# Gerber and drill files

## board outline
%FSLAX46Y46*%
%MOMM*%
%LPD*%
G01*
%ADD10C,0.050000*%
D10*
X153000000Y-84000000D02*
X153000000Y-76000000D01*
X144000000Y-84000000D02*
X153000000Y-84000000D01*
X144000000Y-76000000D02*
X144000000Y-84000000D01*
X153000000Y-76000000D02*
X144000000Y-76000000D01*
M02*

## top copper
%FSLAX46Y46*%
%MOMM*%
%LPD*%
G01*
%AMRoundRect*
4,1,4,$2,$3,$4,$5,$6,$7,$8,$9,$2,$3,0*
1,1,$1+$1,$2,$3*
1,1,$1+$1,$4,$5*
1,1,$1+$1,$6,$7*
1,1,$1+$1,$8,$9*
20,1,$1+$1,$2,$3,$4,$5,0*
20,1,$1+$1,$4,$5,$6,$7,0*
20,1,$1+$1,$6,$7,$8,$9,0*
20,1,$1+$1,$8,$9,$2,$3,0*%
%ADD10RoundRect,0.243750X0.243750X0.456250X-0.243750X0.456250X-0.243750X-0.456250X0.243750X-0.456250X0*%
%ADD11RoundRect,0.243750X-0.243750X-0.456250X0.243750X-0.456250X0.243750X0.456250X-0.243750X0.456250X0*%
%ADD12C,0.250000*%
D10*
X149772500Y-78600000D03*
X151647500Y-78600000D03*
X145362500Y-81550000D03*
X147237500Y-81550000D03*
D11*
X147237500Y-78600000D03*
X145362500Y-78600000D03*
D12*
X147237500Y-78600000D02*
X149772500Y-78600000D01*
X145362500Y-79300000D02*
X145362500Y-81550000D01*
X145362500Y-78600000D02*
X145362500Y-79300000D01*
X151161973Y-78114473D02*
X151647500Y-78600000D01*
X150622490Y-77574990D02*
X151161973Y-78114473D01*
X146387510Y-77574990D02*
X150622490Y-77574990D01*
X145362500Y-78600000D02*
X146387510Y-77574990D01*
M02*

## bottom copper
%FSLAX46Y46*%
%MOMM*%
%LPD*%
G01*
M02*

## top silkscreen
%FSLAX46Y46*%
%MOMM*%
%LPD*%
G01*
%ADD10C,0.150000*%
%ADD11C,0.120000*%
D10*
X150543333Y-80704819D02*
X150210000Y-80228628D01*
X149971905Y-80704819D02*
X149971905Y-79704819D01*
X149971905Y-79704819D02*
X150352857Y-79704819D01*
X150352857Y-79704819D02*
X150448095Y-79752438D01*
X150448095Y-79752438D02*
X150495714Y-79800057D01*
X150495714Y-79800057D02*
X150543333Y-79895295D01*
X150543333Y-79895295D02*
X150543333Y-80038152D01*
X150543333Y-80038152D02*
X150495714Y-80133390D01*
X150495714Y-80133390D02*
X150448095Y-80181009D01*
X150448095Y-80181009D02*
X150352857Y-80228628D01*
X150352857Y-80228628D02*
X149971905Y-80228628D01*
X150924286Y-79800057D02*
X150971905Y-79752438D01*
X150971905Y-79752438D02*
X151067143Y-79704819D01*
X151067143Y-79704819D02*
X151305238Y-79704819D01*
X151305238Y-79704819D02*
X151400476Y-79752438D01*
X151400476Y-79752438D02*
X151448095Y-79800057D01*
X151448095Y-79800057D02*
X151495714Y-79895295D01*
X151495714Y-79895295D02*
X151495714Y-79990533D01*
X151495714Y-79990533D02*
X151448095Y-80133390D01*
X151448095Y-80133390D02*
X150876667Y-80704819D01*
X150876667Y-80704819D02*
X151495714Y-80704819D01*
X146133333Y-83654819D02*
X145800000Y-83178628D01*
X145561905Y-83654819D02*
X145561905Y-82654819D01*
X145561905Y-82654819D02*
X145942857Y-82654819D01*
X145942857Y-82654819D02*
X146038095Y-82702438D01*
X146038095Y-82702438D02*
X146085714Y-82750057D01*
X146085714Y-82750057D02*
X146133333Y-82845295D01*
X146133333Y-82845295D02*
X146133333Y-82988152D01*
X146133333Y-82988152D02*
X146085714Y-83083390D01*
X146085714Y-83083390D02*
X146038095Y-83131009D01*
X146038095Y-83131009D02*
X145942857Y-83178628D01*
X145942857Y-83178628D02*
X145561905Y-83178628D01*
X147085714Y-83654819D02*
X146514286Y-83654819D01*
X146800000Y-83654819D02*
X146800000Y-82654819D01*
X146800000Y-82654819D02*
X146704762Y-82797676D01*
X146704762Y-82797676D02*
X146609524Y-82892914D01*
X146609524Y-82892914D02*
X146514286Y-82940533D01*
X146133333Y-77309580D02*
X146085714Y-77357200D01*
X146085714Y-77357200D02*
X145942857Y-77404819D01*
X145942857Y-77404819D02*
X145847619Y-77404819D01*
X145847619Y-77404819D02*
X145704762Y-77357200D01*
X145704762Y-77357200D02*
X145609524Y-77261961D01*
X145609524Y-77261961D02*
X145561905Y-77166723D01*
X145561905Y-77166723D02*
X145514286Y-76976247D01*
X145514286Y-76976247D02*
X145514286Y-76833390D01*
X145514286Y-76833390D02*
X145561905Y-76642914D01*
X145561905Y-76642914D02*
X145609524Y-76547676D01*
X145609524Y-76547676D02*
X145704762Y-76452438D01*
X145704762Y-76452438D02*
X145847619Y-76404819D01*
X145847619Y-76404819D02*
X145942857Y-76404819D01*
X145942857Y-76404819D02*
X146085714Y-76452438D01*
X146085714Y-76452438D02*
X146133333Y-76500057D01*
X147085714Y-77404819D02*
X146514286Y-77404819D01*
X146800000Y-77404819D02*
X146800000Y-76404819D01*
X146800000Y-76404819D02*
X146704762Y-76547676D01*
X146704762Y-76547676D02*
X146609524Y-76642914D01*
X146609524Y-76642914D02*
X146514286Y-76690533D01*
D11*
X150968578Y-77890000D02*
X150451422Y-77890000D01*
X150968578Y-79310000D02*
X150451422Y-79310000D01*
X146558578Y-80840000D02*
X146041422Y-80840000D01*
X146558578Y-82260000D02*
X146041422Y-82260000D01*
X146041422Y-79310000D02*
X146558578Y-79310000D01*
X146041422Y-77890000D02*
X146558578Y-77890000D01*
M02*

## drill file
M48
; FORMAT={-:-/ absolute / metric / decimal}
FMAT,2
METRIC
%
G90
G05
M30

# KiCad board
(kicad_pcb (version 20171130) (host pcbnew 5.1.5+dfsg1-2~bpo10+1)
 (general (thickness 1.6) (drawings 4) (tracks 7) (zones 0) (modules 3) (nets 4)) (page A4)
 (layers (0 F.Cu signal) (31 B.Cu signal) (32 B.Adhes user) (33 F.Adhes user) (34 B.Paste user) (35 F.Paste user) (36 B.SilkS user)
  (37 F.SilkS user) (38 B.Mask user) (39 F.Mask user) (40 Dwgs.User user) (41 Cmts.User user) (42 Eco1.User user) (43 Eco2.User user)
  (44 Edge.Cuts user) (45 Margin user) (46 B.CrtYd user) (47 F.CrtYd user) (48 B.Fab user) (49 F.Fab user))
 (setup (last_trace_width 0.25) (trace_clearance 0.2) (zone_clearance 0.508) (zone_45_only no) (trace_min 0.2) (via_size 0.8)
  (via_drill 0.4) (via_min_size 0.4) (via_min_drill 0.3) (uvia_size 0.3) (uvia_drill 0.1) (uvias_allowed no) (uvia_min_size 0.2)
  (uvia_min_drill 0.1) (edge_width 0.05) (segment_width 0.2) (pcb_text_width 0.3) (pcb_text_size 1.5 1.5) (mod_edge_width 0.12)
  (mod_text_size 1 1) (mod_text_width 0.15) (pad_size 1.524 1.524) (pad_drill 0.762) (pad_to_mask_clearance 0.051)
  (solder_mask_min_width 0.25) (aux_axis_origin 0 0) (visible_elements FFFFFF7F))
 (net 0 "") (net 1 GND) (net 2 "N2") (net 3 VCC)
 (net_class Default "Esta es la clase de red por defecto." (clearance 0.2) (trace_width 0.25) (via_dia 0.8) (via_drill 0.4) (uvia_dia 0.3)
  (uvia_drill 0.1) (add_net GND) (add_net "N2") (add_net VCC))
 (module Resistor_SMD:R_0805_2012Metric (layer F.Cu) (at 150.71 78.6 180)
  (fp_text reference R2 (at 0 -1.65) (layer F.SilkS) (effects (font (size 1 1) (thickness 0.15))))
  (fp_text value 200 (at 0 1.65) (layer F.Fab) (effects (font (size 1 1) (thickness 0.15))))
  (fp_line (start -0.258578 0.71) (end 0.258578 0.71) (layer F.SilkS) (width 0.12))
  (fp_line (start -0.258578 -0.71) (end 0.258578 -0.71) (layer F.SilkS) (width 0.12))
  (pad 2 smd roundrect (at 0.9375 0 180) (size 0.975 1.4) (layers F.Cu F.Paste F.Mask) (roundrect_rratio 0.25) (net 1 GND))
  (pad 1 smd roundrect (at -0.9375 0 180) (size 0.975 1.4) (layers F.Cu F.Paste F.Mask) (roundrect_rratio 0.25) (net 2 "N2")))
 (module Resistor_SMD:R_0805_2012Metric (layer F.Cu) (at 146.3 81.55 180)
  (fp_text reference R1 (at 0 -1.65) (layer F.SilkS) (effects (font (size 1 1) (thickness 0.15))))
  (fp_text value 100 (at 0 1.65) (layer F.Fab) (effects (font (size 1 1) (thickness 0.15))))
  (fp_line (start -0.258578 0.71) (end 0.258578 0.71) (layer F.SilkS) (width 0.12))
  (fp_line (start -0.258578 -0.71) (end 0.258578 -0.71) (layer F.SilkS) (width 0.12))
  (pad 2 smd roundrect (at 0.9375 0 180) (size 0.975 1.4) (layers F.Cu F.Paste F.Mask) (roundrect_rratio 0.25) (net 2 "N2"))
  (pad 1 smd roundrect (at -0.9375 0 180) (size 0.975 1.4) (layers F.Cu F.Paste F.Mask) (roundrect_rratio 0.25) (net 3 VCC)))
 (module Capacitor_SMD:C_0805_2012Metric (layer F.Cu) (at 146.3 78.6)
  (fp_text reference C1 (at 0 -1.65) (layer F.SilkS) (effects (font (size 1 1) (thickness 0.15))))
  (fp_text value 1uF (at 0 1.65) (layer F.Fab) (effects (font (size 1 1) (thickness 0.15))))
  (fp_line (start -0.258578 0.71) (end 0.258578 0.71) (layer F.SilkS) (width 0.12))
  (fp_line (start -0.258578 -0.71) (end 0.258578 -0.71) (layer F.SilkS) (width 0.12))
  (pad 2 smd roundrect (at 0.9375 0) (size 0.975 1.4) (layers F.Cu F.Paste F.Mask) (roundrect_rratio 0.25) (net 1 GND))
  (pad 1 smd roundrect (at -0.9375 0) (size 0.975 1.4) (layers F.Cu F.Paste F.Mask) (roundrect_rratio 0.25) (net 2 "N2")))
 (gr_line (start 153 84) (end 153 76) (layer Edge.Cuts) (width 0.05))
 (gr_line (start 144 84) (end 153 84) (layer Edge.Cuts) (width 0.05))
 (gr_line (start 144 76) (end 144 84) (layer Edge.Cuts) (width 0.05))
 (gr_line (start 153 76) (end 144 76) (layer Edge.Cuts) (width 0.05))
 (segment (start 147.2375 78.6) (end 149.7725 78.6) (width 0.25) (layer F.Cu) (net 1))
 (segment (start 145.3625 79.3) (end 145.3625 81.55) (width 0.25) (layer F.Cu) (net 2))
 (segment (start 145.3625 78.6) (end 145.3625 79.3) (width 0.25) (layer F.Cu) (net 2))
 (segment (start 151.161973 78.114473) (end 151.6475 78.6) (width 0.25) (layer F.Cu) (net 2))
 (segment (start 150.62249 77.57499) (end 151.161973 78.114473) (width 0.25) (layer F.Cu) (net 2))
 (segment (start 146.38751 77.57499) (end 150.62249 77.57499) (width 0.25) (layer F.Cu) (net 2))
 (segment (start 145.3625 78.6) (end 146.38751 77.57499) (width 0.25) (layer F.Cu) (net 2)))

